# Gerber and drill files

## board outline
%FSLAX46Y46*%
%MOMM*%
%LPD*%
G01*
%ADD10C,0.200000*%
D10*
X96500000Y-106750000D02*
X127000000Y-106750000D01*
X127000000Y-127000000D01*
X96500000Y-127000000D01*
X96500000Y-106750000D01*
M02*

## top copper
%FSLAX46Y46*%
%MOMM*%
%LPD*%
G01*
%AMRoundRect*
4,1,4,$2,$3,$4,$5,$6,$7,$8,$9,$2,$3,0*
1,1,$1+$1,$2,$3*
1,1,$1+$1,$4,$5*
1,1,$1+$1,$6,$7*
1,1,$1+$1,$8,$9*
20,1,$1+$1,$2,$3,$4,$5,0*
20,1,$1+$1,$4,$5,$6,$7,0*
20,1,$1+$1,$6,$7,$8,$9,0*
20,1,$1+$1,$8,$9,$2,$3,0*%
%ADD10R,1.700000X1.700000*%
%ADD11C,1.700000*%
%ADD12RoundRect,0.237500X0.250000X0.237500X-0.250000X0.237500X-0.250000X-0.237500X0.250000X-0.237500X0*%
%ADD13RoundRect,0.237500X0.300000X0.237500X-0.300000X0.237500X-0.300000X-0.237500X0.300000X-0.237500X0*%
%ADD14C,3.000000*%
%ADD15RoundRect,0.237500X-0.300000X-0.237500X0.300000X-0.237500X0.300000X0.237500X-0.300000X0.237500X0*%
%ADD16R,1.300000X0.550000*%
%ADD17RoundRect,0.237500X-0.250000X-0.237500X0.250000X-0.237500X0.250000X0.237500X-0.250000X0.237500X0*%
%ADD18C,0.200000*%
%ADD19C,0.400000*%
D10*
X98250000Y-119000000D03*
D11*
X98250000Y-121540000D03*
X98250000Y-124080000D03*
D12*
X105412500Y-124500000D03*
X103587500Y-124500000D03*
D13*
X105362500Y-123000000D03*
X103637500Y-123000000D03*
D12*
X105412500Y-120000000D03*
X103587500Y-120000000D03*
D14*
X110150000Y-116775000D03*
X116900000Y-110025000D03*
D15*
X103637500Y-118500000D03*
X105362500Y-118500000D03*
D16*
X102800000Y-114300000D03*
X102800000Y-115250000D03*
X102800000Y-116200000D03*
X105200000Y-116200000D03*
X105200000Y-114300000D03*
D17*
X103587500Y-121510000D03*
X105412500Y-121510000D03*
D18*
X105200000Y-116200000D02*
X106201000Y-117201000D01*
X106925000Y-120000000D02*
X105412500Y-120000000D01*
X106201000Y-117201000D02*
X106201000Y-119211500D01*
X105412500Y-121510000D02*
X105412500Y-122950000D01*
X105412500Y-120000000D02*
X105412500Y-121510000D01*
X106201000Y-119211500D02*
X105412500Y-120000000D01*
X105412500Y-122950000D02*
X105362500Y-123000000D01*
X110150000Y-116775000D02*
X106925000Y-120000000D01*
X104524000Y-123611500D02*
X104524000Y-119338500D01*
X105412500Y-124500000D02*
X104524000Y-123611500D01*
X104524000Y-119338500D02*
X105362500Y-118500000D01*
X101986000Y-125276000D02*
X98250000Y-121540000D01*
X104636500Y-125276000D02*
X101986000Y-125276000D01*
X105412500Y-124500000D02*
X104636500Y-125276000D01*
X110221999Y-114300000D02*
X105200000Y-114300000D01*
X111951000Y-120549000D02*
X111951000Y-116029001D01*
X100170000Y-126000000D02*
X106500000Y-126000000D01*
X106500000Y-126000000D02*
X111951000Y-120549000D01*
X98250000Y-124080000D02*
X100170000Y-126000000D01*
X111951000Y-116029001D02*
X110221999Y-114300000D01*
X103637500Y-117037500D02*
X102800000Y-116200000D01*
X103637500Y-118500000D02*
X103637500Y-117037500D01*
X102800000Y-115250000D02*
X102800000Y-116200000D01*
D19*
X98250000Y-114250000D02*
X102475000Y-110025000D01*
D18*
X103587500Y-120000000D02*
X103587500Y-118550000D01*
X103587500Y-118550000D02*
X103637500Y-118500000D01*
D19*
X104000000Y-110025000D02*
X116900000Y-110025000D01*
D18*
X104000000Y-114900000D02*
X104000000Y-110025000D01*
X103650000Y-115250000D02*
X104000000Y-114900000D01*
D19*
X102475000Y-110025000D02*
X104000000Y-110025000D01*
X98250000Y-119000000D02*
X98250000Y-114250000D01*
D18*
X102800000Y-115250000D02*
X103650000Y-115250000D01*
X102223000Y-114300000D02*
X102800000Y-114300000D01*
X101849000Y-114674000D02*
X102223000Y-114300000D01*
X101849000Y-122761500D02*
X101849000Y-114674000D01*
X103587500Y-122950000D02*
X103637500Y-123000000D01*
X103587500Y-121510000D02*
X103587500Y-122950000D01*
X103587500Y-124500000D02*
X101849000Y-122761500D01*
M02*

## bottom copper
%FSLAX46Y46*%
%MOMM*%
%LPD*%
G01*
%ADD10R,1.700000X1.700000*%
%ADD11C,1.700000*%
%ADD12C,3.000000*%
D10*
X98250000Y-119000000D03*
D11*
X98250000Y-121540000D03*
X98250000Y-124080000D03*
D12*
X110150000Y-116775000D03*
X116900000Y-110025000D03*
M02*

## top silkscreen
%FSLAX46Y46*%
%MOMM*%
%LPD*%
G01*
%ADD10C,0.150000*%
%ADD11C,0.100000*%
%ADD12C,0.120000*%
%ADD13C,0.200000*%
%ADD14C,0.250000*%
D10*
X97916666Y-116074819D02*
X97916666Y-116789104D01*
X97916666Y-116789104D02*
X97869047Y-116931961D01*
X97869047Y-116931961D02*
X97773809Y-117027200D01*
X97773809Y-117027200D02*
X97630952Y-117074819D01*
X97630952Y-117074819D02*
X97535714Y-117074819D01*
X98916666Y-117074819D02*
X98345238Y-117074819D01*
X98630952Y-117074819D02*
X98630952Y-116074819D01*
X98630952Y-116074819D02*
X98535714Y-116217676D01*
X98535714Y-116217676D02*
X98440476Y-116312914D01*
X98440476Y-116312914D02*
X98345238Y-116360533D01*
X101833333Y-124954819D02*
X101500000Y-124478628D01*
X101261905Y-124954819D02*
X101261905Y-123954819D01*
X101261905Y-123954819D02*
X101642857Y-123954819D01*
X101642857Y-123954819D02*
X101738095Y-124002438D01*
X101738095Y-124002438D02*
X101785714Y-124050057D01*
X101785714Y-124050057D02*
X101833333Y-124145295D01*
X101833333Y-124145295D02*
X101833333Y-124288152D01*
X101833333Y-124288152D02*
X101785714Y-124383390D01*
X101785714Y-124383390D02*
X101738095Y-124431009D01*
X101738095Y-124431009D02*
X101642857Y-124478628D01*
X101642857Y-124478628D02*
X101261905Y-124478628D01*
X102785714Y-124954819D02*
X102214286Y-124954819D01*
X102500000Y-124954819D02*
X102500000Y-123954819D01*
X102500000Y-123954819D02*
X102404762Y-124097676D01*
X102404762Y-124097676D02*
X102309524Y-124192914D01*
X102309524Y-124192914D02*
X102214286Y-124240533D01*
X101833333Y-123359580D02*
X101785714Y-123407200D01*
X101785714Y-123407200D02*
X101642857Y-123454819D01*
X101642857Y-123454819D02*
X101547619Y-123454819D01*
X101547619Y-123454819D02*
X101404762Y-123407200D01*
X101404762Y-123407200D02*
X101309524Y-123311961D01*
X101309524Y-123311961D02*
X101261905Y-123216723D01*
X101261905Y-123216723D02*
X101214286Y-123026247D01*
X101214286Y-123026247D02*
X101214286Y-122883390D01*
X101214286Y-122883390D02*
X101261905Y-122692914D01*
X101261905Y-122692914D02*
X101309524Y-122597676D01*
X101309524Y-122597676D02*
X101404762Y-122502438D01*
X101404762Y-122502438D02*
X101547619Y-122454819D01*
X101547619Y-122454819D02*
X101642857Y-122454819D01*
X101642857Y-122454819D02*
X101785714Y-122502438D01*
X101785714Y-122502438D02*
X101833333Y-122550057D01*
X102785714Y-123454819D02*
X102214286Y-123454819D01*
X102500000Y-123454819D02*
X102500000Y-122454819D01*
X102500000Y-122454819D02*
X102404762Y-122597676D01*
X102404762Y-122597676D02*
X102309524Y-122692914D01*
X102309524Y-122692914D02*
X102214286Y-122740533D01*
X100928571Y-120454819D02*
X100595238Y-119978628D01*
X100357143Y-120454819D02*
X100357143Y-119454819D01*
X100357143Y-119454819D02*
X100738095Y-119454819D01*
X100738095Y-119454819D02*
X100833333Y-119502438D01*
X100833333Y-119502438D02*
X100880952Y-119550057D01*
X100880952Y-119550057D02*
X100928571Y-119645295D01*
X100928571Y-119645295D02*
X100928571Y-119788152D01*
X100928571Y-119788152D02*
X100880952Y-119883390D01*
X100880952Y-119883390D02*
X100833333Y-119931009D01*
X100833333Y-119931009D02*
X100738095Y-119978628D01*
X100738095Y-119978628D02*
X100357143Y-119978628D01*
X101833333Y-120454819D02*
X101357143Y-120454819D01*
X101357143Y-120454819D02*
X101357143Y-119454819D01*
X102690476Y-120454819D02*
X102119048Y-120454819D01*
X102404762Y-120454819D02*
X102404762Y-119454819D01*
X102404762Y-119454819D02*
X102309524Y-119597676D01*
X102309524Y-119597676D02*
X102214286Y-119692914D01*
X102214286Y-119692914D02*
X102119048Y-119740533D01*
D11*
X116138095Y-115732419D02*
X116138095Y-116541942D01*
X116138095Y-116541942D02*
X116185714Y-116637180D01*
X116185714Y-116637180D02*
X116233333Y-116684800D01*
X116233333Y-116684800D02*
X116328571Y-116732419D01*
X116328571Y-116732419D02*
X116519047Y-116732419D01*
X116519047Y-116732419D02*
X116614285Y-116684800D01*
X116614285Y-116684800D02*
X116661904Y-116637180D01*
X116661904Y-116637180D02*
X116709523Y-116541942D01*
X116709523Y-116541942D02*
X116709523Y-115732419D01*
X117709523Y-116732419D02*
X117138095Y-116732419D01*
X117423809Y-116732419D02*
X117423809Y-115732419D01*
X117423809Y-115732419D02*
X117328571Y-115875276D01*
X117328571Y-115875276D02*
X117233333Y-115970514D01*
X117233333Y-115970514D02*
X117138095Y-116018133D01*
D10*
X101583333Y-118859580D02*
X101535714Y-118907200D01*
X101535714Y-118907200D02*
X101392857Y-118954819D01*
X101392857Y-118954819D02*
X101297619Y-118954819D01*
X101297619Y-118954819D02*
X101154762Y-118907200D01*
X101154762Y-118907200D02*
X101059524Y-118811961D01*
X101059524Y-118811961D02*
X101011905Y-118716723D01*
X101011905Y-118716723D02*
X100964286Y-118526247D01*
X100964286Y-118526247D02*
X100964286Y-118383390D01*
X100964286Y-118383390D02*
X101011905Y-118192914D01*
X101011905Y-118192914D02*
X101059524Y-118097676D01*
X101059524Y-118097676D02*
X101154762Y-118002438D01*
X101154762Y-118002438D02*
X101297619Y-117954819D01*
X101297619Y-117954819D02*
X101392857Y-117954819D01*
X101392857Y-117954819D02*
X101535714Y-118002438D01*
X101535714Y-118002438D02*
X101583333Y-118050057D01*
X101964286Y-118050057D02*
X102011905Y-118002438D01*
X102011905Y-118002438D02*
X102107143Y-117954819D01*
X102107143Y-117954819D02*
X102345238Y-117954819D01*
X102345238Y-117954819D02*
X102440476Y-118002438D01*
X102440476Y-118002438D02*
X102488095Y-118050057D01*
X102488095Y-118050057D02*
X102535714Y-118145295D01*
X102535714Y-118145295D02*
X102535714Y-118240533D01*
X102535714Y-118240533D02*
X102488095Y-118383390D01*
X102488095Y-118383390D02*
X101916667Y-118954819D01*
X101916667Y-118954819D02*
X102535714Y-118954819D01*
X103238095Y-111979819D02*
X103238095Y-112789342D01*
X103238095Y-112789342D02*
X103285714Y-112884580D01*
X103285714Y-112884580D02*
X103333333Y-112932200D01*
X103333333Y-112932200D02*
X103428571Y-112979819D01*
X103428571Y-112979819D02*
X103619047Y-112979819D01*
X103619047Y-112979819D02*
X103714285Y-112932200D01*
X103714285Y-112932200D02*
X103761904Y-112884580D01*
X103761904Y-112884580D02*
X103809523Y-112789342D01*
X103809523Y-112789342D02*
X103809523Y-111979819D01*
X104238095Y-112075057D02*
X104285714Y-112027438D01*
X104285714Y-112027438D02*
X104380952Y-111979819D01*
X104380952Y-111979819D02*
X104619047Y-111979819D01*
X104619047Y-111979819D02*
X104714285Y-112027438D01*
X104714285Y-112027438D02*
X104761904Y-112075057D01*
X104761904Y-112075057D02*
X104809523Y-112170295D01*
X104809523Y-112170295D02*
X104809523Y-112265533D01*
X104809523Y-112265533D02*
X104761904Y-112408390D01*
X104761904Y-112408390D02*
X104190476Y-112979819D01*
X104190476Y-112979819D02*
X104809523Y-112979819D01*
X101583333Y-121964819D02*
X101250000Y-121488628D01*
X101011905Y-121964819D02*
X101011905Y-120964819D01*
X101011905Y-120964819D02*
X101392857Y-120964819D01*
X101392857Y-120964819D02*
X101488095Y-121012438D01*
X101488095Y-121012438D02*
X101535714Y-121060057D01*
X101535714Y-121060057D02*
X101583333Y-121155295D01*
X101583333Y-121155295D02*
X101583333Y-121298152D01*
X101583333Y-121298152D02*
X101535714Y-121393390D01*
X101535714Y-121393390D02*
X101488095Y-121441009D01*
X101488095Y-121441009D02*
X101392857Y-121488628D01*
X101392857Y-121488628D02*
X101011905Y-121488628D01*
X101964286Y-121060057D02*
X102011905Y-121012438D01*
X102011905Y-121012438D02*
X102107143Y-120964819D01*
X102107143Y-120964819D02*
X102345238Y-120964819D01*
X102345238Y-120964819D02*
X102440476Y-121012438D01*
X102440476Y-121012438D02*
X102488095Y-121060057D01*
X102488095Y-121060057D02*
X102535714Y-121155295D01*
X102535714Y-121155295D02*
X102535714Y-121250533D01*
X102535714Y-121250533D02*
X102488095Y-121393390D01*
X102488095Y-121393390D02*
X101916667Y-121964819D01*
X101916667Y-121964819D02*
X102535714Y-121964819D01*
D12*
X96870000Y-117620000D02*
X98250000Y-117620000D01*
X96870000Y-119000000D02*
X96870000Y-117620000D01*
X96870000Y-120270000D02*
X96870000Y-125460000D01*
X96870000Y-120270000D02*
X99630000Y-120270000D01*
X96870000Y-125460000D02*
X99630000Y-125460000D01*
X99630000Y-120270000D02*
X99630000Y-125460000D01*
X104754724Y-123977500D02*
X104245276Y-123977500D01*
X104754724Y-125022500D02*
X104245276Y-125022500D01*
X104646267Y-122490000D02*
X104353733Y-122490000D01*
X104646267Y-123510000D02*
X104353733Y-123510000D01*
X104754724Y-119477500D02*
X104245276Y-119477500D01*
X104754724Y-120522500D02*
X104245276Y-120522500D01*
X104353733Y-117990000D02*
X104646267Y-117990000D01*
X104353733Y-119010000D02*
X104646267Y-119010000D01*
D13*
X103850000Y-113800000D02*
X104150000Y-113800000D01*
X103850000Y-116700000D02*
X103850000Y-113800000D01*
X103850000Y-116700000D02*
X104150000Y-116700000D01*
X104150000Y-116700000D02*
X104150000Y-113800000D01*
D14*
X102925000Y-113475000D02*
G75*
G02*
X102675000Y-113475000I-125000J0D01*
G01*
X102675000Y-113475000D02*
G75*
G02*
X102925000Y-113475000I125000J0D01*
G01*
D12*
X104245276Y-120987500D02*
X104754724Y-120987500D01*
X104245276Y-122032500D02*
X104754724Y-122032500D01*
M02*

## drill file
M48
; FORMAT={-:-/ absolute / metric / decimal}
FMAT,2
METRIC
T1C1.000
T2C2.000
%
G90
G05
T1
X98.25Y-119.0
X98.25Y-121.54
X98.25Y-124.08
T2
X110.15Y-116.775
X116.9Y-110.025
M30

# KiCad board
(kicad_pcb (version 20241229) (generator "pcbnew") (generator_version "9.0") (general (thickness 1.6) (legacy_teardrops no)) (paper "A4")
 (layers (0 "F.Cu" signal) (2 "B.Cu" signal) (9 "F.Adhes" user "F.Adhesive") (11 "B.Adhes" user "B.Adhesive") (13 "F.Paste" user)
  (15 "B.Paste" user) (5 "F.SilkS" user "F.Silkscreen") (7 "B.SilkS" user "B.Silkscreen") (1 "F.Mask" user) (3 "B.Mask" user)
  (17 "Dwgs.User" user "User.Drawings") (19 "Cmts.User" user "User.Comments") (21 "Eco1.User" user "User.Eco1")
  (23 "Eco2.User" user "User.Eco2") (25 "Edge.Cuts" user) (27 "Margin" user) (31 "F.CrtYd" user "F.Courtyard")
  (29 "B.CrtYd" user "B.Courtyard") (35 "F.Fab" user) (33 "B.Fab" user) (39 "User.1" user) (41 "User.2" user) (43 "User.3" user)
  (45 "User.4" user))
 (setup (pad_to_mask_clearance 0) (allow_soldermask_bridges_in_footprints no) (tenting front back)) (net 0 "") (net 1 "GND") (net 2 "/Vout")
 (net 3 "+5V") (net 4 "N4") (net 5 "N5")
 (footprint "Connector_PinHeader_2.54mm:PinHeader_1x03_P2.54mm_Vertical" (layer "F.Cu") (at 98.25 119)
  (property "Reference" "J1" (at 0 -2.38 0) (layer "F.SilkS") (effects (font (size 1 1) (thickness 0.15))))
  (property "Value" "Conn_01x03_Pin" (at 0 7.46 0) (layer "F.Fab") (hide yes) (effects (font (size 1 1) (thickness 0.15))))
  (fp_line (start -1.38 -1.38) (end 0 -1.38) (stroke (width 0.12) (type solid)) (layer "F.SilkS"))
  (fp_line (start -1.38 0) (end -1.38 -1.38) (stroke (width 0.12) (type solid)) (layer "F.SilkS"))
  (fp_line (start -1.38 1.27) (end -1.38 6.46) (stroke (width 0.12) (type solid)) (layer "F.SilkS"))
  (fp_line (start -1.38 1.27) (end 1.38 1.27) (stroke (width 0.12) (type solid)) (layer "F.SilkS"))
  (fp_line (start -1.38 6.46) (end 1.38 6.46) (stroke (width 0.12) (type solid)) (layer "F.SilkS"))
  (fp_line (start 1.38 1.27) (end 1.38 6.46) (stroke (width 0.12) (type solid)) (layer "F.SilkS"))
  (pad "1" thru_hole rect (at 0 0) (size 1.7 1.7) (drill 1) (layers "*.Cu" "*.Mask") (remove_unused_layers no) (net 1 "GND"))
  (pad "2" thru_hole circle (at 0 2.54) (size 1.7 1.7) (drill 1) (layers "*.Cu" "*.Mask") (remove_unused_layers no) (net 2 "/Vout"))
  (pad "3" thru_hole circle (at 0 5.08) (size 1.7 1.7) (drill 1) (layers "*.Cu" "*.Mask") (remove_unused_layers no) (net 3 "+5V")))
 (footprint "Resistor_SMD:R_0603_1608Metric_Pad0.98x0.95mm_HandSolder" (layer "F.Cu") (at 104.5 124.5 180)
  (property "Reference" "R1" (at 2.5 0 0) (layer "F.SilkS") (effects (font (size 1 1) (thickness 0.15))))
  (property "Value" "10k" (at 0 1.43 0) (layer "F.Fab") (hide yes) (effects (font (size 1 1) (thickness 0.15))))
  (fp_line (start -0.254724 0.5225) (end 0.254724 0.5225) (stroke (width 0.12) (type solid)) (layer "F.SilkS"))
  (fp_line (start -0.254724 -0.5225) (end 0.254724 -0.5225) (stroke (width 0.12) (type solid)) (layer "F.SilkS"))
  (pad "1" smd roundrect (at -0.9125 0 180) (size 0.975 0.95) (layers "F.Cu" "F.Mask" "F.Paste") (roundrect_rratio 0.25) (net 2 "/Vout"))
  (pad "2" smd roundrect (at 0.9125 0 180) (size 0.975 0.95) (layers "F.Cu" "F.Mask" "F.Paste") (roundrect_rratio 0.25) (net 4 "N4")))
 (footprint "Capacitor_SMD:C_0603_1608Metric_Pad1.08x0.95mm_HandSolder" (layer "F.Cu") (at 104.5 123 180)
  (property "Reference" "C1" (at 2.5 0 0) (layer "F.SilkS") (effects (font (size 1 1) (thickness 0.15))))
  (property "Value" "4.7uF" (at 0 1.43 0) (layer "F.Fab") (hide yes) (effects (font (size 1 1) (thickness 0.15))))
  (fp_line (start -0.146267 0.51) (end 0.146267 0.51) (stroke (width 0.12) (type solid)) (layer "F.SilkS"))
  (fp_line (start -0.146267 -0.51) (end 0.146267 -0.51) (stroke (width 0.12) (type solid)) (layer "F.SilkS"))
  (pad "1" smd roundrect (at -0.8625 0 180) (size 1.075 0.95) (layers "F.Cu" "F.Mask" "F.Paste") (roundrect_rratio 0.25) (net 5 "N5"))
  (pad "2" smd roundrect (at 0.8625 0 180) (size 1.075 0.95) (layers "F.Cu" "F.Mask" "F.Paste") (roundrect_rratio 0.25) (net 4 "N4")))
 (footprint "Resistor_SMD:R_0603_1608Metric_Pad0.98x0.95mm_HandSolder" (layer "F.Cu") (at 104.5 120 180)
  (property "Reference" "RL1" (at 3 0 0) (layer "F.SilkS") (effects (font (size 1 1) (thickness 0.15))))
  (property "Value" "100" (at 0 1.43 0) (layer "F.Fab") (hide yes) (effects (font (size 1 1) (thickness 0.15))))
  (fp_line (start -0.254724 0.5225) (end 0.254724 0.5225) (stroke (width 0.12) (type solid)) (layer "F.SilkS"))
  (fp_line (start -0.254724 -0.5225) (end 0.254724 -0.5225) (stroke (width 0.12) (type solid)) (layer "F.SilkS"))
  (pad "1" smd roundrect (at -0.9125 0 180) (size 0.975 0.95) (layers "F.Cu" "F.Mask" "F.Paste") (roundrect_rratio 0.25) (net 5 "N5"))
  (pad "2" smd roundrect (at 0.9125 0 180) (size 0.975 0.95) (layers "F.Cu" "F.Mask" "F.Paste") (roundrect_rratio 0.25) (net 1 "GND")))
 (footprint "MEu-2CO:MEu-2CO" (layer "F.Cu") (at 116.9 116.775)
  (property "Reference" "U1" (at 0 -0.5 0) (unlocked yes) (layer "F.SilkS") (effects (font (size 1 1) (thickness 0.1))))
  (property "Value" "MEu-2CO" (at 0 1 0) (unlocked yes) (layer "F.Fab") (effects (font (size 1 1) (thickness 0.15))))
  (pad "1" thru_hole circle (at -6.75 0) (size 3 3) (drill 2) (layers "*.Cu" "*.Mask") (remove_unused_layers no) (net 5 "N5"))
  (pad "2" thru_hole circle (at 0 -6.75) (size 3 3) (drill 2) (layers "*.Cu" "*.Mask") (remove_unused_layers no) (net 1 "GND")))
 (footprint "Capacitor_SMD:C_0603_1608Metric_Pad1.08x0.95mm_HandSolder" (layer "F.Cu") (at 104.5 118.5)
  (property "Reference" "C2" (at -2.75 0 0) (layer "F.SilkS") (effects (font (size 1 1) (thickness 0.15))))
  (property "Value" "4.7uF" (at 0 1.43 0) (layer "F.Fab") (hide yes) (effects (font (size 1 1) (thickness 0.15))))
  (fp_line (start -0.146267 -0.51) (end 0.146267 -0.51) (stroke (width 0.12) (type solid)) (layer "F.SilkS"))
  (fp_line (start -0.146267 0.51) (end 0.146267 0.51) (stroke (width 0.12) (type solid)) (layer "F.SilkS"))
  (pad "1" smd roundrect (at -0.8625 0) (size 1.075 0.95) (layers "F.Cu" "F.Mask" "F.Paste") (roundrect_rratio 0.25) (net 1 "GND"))
  (pad "2" smd roundrect (at 0.8625 0) (size 1.075 0.95) (layers "F.Cu" "F.Mask" "F.Paste") (roundrect_rratio 0.25) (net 2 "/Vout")))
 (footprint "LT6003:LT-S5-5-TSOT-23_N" (layer "F.Cu") (at 104 115.25)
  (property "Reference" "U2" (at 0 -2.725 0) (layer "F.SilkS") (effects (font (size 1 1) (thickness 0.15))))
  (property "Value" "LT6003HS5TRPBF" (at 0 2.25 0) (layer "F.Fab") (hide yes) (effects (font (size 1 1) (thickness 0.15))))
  (fp_line (start -0.15 -1.45) (end 0.15 -1.45) (stroke (width 0.2) (type solid)) (layer "F.SilkS"))
  (fp_line (start -0.15 1.45) (end -0.15 -1.45) (stroke (width 0.2) (type solid)) (layer "F.SilkS"))
  (fp_line (start -0.15 1.45) (end 0.15 1.45) (stroke (width 0.2) (type solid)) (layer "F.SilkS"))
  (fp_line (start 0.15 1.45) (end 0.15 -1.45) (stroke (width 0.2) (type solid)) (layer "F.SilkS"))
  (fp_circle (center -1.2 -1.775) (end -1.2 -1.9) (stroke (width 0.25) (type solid)) (fill no) (layer "F.SilkS"))
  (pad "1" smd rect (at -1.2 -0.95 90) (size 0.55 1.3) (layers "F.Cu" "F.Mask" "F.Paste") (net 4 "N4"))
  (pad "2" smd rect (at -1.2 0 90) (size 0.55 1.3) (layers "F.Cu" "F.Mask" "F.Paste") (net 1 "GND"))
  (pad "3" smd rect (at -1.2 0.95 90) (size 0.55 1.3) (layers "F.Cu" "F.Mask" "F.Paste") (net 1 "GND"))
  (pad "4" smd rect (at 1.2 0.95 90) (size 0.55 1.3) (layers "F.Cu" "F.Mask" "F.Paste") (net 5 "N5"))
  (pad "5" smd rect (at 1.2 -0.95 90) (size 0.55 1.3) (layers "F.Cu" "F.Mask" "F.Paste") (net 3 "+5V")))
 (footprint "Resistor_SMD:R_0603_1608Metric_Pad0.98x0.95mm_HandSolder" (layer "F.Cu") (at 104.5 121.51)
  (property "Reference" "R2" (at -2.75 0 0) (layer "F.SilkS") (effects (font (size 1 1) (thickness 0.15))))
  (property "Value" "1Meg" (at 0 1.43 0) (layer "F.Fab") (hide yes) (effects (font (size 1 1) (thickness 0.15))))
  (fp_line (start -0.254724 -0.5225) (end 0.254724 -0.5225) (stroke (width 0.12) (type solid)) (layer "F.SilkS"))
  (fp_line (start -0.254724 0.5225) (end 0.254724 0.5225) (stroke (width 0.12) (type solid)) (layer "F.SilkS"))
  (pad "1" smd roundrect (at -0.9125 0) (size 0.975 0.95) (layers "F.Cu" "F.Mask" "F.Paste") (roundrect_rratio 0.25) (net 4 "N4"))
  (pad "2" smd roundrect (at 0.9125 0) (size 0.975 0.95) (layers "F.Cu" "F.Mask" "F.Paste") (roundrect_rratio 0.25) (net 5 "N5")))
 (gr_rect (start 96.5 106.75) (end 127 127) (stroke (width 0.2) (type solid)) (fill no) (layer "Edge.Cuts"))
 (segment (start 105.2 116.2) (end 106.201 117.201) (width 0.2) (layer "F.Cu") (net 5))
 (segment (start 106.925 120) (end 105.4125 120) (width 0.2) (layer "F.Cu") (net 5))
 (segment (start 106.201 117.201) (end 106.201 119.2115) (width 0.2) (layer "F.Cu") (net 5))
 (segment (start 105.4125 121.51) (end 105.4125 122.95) (width 0.2) (layer "F.Cu") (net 5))
 (segment (start 105.4125 120) (end 105.4125 121.51) (width 0.2) (layer "F.Cu") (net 5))
 (segment (start 106.201 119.2115) (end 105.4125 120) (width 0.2) (layer "F.Cu") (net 5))
 (segment (start 105.4125 122.95) (end 105.3625 123) (width 0.2) (layer "F.Cu") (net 5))
 (segment (start 110.15 116.775) (end 106.925 120) (width 0.2) (layer "F.Cu") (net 5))
 (segment (start 104.524 123.6115) (end 104.524 119.3385) (width 0.2) (layer "F.Cu") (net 2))
 (segment (start 105.4125 124.5) (end 104.524 123.6115) (width 0.2) (layer "F.Cu") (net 2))
 (segment (start 104.524 119.3385) (end 105.3625 118.5) (width 0.2) (layer "F.Cu") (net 2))
 (segment (start 101.986 125.276) (end 98.25 121.54) (width 0.2) (layer "F.Cu") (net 2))
 (segment (start 104.6365 125.276) (end 101.986 125.276) (width 0.2) (layer "F.Cu") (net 2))
 (segment (start 105.4125 124.5) (end 104.6365 125.276) (width 0.2) (layer "F.Cu") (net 2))
 (segment (start 110.221999 114.3) (end 105.2 114.3) (width 0.2) (layer "F.Cu") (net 3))
 (segment (start 111.951 120.549) (end 111.951 116.029001) (width 0.2) (layer "F.Cu") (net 3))
 (segment (start 100.17 126) (end 106.5 126) (width 0.2) (layer "F.Cu") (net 3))
 (segment (start 106.5 126) (end 111.951 120.549) (width 0.2) (layer "F.Cu") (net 3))
 (segment (start 98.25 124.08) (end 100.17 126) (width 0.2) (layer "F.Cu") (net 3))
 (segment (start 111.951 116.029001) (end 110.221999 114.3) (width 0.2) (layer "F.Cu") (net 3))
 (segment (start 103.6375 117.0375) (end 102.8 116.2) (width 0.2) (layer "F.Cu") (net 1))
 (segment (start 103.6375 118.5) (end 103.6375 117.0375) (width 0.2) (layer "F.Cu") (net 1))
 (segment (start 102.8 115.25) (end 102.8 116.2) (width 0.2) (layer "F.Cu") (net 1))
 (segment (start 98.25 114.25) (end 102.475 110.025) (width 0.4) (layer "F.Cu") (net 1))
 (segment (start 103.5875 120) (end 103.5875 118.55) (width 0.2) (layer "F.Cu") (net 1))
 (segment (start 103.5875 118.55) (end 103.6375 118.5) (width 0.2) (layer "F.Cu") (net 1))
 (segment (start 104 110.025) (end 116.9 110.025) (width 0.4) (layer "F.Cu") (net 1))
 (segment (start 104 114.9) (end 104 110.025) (width 0.2) (layer "F.Cu") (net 1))
 (segment (start 103.65 115.25) (end 104 114.9) (width 0.2) (layer "F.Cu") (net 1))
 (segment (start 102.475 110.025) (end 104 110.025) (width 0.4) (layer "F.Cu") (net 1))
 (segment (start 98.25 119) (end 98.25 114.25) (width 0.4) (layer "F.Cu") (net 1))
 (segment (start 102.8 115.25) (end 103.65 115.25) (width 0.2) (layer "F.Cu") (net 1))
 (segment (start 102.223 114.3) (end 102.8 114.3) (width 0.2) (layer "F.Cu") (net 4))
 (segment (start 101.849 114.674) (end 102.223 114.3) (width 0.2) (layer "F.Cu") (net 4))
 (segment (start 101.849 122.7615) (end 101.849 114.674) (width 0.2) (layer "F.Cu") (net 4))
 (segment (start 103.5875 122.95) (end 103.6375 123) (width 0.2) (layer "F.Cu") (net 4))
 (segment (start 103.5875 121.51) (end 103.5875 122.95) (width 0.2) (layer "F.Cu") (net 4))
 (segment (start 103.5875 124.5) (end 101.849 122.7615) (width 0.2) (layer "F.Cu") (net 4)))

